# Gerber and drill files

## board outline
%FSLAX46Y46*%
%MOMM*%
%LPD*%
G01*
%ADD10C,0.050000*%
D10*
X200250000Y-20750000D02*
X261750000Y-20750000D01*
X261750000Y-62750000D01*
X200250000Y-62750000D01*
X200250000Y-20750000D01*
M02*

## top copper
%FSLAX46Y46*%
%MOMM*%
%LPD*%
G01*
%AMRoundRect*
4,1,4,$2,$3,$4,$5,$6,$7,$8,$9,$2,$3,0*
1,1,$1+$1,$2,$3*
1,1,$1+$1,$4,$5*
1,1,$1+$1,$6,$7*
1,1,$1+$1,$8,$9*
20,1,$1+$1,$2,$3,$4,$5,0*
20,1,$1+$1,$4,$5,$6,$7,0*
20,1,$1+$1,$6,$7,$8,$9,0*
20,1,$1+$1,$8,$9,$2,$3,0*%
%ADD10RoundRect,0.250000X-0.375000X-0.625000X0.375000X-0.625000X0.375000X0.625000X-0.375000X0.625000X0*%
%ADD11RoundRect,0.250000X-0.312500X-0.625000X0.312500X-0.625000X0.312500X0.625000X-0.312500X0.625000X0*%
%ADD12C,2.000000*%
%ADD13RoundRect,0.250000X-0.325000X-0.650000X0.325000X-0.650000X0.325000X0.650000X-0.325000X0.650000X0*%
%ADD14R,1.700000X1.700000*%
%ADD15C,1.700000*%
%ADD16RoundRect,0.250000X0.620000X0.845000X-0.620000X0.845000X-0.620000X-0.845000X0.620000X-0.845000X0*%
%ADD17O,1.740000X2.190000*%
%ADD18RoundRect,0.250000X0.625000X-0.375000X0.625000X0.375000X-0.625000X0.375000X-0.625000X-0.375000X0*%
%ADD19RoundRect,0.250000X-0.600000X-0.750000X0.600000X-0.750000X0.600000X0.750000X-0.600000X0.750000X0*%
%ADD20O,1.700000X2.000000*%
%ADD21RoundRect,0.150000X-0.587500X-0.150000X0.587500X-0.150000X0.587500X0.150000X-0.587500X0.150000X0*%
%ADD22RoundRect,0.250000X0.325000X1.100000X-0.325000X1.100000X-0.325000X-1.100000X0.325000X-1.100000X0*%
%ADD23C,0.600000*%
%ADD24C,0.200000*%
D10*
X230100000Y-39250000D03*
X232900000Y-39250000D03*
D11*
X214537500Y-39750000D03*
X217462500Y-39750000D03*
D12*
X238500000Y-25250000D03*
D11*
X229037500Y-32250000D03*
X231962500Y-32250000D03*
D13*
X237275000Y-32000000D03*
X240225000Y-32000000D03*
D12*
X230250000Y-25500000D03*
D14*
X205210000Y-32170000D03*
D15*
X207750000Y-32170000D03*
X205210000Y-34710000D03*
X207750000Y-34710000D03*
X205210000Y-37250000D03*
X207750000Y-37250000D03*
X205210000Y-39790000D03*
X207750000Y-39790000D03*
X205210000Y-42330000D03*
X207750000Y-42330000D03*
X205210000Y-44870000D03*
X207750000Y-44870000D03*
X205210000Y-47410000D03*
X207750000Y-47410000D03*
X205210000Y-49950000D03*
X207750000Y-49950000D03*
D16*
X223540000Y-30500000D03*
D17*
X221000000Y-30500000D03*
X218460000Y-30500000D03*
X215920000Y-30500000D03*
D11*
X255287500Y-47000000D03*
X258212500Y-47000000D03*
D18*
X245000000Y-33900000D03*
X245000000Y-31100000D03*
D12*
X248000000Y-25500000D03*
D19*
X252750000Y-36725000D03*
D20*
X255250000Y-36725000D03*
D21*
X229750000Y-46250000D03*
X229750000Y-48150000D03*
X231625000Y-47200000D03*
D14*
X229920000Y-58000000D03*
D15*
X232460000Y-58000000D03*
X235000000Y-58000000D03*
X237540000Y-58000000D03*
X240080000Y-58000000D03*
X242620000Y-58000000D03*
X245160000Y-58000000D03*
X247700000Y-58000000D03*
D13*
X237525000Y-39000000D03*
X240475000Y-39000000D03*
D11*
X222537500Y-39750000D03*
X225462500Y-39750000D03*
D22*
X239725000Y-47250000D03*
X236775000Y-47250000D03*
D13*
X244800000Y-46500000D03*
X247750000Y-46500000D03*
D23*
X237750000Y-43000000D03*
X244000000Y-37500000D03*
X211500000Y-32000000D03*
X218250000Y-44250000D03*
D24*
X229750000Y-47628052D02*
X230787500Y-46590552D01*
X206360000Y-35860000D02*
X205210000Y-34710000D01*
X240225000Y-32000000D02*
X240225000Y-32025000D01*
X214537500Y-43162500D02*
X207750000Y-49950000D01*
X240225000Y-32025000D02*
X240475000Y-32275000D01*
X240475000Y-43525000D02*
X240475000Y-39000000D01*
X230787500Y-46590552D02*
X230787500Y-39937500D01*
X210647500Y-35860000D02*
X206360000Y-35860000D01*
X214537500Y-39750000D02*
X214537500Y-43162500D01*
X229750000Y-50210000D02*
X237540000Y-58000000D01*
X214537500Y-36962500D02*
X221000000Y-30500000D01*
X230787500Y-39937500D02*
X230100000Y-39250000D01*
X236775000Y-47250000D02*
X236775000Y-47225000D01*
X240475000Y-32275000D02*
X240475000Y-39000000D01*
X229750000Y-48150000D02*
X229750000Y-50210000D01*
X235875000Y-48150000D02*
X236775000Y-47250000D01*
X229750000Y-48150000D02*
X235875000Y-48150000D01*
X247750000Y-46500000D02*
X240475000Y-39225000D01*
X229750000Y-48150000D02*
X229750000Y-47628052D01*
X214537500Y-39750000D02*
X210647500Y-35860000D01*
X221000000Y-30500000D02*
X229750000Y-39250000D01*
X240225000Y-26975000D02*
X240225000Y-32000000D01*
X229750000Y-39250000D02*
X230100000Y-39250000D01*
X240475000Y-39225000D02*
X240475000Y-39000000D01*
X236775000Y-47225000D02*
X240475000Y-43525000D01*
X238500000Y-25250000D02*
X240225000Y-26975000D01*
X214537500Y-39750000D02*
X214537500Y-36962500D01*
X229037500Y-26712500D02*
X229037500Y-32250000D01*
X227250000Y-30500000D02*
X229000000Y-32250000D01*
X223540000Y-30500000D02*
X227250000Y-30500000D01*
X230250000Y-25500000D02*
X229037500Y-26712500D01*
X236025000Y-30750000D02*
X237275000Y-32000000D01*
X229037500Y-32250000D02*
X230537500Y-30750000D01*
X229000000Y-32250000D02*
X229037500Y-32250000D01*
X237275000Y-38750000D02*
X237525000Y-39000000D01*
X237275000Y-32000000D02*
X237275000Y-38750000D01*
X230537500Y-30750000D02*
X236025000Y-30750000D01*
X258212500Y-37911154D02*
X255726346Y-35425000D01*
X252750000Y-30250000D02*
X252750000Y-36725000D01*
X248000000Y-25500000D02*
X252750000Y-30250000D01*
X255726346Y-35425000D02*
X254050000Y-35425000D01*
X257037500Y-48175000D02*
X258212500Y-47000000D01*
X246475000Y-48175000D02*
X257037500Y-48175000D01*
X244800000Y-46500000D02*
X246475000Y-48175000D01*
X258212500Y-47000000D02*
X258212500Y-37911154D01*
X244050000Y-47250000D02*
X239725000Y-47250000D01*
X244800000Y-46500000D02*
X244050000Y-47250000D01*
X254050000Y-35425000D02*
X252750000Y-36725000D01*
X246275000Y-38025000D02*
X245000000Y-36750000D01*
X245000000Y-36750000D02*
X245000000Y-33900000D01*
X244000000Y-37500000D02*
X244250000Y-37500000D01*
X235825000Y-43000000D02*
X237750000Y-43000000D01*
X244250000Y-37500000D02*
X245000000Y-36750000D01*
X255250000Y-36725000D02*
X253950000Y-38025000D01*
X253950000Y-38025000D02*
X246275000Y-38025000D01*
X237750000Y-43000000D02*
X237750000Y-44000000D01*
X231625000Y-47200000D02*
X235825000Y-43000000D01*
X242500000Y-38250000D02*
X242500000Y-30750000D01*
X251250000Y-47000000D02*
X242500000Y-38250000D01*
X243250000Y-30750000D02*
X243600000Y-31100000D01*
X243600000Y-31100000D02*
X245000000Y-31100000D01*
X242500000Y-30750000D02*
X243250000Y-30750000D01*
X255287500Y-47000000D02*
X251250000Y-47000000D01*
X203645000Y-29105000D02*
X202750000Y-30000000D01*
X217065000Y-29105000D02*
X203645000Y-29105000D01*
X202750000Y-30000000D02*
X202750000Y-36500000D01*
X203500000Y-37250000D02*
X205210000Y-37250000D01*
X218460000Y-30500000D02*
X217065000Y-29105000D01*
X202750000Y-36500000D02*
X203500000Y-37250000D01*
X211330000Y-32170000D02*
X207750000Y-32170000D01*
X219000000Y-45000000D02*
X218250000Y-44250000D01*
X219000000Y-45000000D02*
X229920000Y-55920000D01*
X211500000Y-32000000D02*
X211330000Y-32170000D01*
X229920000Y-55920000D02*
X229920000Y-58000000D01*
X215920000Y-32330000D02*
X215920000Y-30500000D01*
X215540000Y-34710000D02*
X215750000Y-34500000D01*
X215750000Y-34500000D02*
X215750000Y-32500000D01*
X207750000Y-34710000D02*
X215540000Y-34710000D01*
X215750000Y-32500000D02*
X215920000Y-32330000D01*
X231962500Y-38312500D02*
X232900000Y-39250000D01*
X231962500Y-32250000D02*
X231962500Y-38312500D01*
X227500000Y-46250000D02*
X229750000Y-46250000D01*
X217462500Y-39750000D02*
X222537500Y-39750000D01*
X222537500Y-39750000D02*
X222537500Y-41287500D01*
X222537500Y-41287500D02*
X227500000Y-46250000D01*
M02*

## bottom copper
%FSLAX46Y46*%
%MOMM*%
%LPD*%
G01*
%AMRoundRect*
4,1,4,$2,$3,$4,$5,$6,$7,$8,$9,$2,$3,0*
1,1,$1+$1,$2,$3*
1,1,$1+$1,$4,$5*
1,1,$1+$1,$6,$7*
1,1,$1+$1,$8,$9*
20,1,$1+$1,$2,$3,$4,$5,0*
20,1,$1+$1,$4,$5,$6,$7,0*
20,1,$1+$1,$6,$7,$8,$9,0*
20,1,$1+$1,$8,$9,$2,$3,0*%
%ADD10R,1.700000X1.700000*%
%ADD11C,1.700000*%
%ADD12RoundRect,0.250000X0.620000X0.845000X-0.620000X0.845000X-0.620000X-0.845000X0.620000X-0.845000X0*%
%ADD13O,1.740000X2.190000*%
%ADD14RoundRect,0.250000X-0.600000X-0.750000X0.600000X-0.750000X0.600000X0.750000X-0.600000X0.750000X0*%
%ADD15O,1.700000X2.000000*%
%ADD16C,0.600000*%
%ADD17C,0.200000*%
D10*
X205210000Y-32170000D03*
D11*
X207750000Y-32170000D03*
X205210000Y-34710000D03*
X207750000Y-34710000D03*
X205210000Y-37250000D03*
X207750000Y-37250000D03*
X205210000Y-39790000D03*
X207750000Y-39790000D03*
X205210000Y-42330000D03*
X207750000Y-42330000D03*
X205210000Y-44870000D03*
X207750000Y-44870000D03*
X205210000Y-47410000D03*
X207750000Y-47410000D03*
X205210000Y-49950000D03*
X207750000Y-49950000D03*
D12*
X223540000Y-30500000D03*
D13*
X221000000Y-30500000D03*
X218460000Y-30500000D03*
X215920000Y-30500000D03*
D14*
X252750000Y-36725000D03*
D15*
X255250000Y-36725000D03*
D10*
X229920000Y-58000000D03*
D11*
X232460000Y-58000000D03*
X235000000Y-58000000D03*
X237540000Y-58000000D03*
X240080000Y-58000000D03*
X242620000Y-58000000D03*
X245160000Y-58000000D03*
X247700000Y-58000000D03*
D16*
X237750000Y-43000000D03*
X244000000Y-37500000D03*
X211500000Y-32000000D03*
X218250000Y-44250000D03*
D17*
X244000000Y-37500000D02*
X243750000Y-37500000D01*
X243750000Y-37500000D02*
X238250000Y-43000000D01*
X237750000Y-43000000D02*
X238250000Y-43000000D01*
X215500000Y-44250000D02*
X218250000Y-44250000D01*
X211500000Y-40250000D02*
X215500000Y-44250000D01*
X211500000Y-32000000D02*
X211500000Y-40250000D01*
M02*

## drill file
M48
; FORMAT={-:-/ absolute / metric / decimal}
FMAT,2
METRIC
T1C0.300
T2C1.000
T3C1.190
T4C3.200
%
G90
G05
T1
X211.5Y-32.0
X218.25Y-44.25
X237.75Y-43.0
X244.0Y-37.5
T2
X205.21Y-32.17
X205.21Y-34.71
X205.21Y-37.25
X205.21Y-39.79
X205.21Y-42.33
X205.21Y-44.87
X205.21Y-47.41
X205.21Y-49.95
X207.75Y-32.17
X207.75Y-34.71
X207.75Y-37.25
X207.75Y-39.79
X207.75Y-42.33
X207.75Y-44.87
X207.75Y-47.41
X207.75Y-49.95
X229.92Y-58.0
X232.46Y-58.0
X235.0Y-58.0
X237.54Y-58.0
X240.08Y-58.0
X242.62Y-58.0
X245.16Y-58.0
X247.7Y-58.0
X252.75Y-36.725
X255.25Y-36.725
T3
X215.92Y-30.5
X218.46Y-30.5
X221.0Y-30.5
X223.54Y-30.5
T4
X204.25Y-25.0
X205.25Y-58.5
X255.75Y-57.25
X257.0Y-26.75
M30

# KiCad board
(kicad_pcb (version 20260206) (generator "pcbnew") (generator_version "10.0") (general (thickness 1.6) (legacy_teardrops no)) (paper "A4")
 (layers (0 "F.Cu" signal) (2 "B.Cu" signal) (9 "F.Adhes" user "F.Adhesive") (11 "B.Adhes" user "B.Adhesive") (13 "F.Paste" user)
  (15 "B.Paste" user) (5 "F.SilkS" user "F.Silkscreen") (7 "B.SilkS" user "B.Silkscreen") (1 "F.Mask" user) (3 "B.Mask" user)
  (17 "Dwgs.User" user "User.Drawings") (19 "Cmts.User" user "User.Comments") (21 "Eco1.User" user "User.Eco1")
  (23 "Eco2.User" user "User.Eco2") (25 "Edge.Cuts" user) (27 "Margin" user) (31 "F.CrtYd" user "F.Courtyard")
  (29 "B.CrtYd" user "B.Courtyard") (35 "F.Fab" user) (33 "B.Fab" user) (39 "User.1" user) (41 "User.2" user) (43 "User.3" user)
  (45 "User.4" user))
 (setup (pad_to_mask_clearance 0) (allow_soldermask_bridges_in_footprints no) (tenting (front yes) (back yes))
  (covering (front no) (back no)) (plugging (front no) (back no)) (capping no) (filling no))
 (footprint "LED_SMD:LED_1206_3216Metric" (layer "F.Cu") (at 231.5 39.25)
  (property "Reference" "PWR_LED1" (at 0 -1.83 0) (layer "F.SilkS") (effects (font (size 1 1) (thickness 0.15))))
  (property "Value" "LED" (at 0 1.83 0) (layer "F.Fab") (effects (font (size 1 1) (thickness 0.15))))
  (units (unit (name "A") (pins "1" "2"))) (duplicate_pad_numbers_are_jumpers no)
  (pad "1" smd roundrect (at -1.4 0) (size 1.25 1.75) (layers "F.Cu" "F.Mask" "F.Paste") (roundrect_rratio 0.2) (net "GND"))
  (pad "2" smd roundrect (at 1.4 0) (size 1.25 1.75) (layers "F.Cu" "F.Mask" "F.Paste") (roundrect_rratio 0.2) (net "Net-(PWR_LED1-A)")))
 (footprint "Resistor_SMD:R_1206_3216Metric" (layer "F.Cu") (at 216 39.75)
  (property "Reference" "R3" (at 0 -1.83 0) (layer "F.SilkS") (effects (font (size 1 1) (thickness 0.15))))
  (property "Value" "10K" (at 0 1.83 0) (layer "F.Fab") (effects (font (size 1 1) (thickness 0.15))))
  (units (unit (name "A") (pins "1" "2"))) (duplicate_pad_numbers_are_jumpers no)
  (pad "1" smd roundrect (at -1.4625 0) (size 1.125 1.75) (layers "F.Cu" "F.Mask" "F.Paste") (roundrect_rratio 0.222222) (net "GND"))
  (pad "2" smd roundrect (at 1.4625 0) (size 1.125 1.75) (layers "F.Cu" "F.Mask" "F.Paste") (roundrect_rratio 0.222222) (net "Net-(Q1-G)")))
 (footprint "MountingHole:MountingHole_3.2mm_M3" (layer "F.Cu") (at 255.75 57.25)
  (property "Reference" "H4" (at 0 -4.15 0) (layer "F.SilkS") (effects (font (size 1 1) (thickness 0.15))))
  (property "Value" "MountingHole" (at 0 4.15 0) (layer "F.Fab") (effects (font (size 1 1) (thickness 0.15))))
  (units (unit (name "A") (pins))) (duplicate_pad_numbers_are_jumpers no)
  (pad "" np_thru_hole circle (at 0 0) (size 3.2 3.2) (drill 3.2) (layers "*.Cu" "*.Mask")))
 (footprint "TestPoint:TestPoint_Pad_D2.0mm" (layer "F.Cu") (at 238.5 25.25 180)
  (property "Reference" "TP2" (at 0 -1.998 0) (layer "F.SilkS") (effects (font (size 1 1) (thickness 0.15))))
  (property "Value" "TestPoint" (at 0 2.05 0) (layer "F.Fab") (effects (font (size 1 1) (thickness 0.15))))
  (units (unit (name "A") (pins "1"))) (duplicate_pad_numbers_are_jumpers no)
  (pad "1" smd circle (at 0 0 180) (size 2 2) (layers "F.Cu" "F.Mask") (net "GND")))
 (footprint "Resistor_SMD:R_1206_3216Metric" (layer "F.Cu") (at 230.5 32.25)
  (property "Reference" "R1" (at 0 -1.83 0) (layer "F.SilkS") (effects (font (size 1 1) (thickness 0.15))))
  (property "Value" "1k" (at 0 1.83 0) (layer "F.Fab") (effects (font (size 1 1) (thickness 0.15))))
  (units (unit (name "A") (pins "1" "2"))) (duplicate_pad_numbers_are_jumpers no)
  (pad "1" smd roundrect (at -1.4625 0) (size 1.125 1.75) (layers "F.Cu" "F.Mask" "F.Paste") (roundrect_rratio 0.222222) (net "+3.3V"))
  (pad "2" smd roundrect (at 1.4625 0) (size 1.125 1.75) (layers "F.Cu" "F.Mask" "F.Paste") (roundrect_rratio 0.222222)
   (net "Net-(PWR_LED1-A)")))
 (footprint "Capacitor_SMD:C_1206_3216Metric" (layer "F.Cu") (at 238.75 32)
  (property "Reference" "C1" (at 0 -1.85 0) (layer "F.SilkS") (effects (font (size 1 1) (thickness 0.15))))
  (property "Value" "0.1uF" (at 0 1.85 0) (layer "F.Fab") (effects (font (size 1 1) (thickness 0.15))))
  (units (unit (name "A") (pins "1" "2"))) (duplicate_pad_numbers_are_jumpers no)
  (pad "1" smd roundrect (at -1.475 0) (size 1.15 1.8) (layers "F.Cu" "F.Mask" "F.Paste") (roundrect_rratio 0.217391) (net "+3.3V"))
  (pad "2" smd roundrect (at 1.475 0) (size 1.15 1.8) (layers "F.Cu" "F.Mask" "F.Paste") (roundrect_rratio 0.217391) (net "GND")))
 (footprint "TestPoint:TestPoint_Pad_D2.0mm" (layer "F.Cu") (at 230.25 25.5 180)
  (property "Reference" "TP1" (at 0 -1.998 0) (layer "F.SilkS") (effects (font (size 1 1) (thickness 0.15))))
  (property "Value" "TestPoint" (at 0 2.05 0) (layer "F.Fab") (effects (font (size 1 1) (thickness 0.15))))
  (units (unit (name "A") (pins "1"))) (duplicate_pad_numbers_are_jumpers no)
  (pad "1" smd circle (at 0 0 180) (size 2 2) (layers "F.Cu" "F.Mask") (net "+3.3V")))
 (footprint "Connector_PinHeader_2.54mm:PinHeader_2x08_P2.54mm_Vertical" (layer "F.Cu") (at 205.21 32.17)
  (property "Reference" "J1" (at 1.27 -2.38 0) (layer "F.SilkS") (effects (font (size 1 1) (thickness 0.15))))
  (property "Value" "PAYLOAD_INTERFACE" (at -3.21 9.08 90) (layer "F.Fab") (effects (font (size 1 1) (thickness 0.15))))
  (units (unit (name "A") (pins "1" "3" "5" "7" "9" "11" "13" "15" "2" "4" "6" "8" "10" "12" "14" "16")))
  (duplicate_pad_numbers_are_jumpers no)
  (pad "1" thru_hole rect (at 0 0) (size 1.7 1.7) (drill 1) (layers "*.Cu" "*.Mask") (remove_unused_layers no) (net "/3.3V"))
  (pad "2" thru_hole circle (at 2.54 0) (size 1.7 1.7) (drill 1) (layers "*.Cu" "*.Mask") (remove_unused_layers no) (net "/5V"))
  (pad "3" thru_hole circle (at 0 2.54) (size 1.7 1.7) (drill 1) (layers "*.Cu" "*.Mask") (remove_unused_layers no) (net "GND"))
  (pad "4" thru_hole circle (at 2.54 2.54) (size 1.7 1.7) (drill 1) (layers "*.Cu" "*.Mask") (remove_unused_layers no) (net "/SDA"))
  (pad "5" thru_hole circle (at 0 5.08) (size 1.7 1.7) (drill 1) (layers "*.Cu" "*.Mask") (remove_unused_layers no) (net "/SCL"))
  (pad "6" thru_hole circle (at 2.54 5.08) (size 1.7 1.7) (drill 1) (layers "*.Cu" "*.Mask") (remove_unused_layers no) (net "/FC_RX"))
  (pad "7" thru_hole circle (at 0 7.62) (size 1.7 1.7) (drill 1) (layers "*.Cu" "*.Mask") (remove_unused_layers no) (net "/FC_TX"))
  (pad "8" thru_hole circle (at 2.54 7.62) (size 1.7 1.7) (drill 1) (layers "*.Cu" "*.Mask") (remove_unused_layers no) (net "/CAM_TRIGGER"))
  (pad "9" thru_hole circle (at 0 10.16) (size 1.7 1.7) (drill 1) (layers "*.Cu" "*.Mask") (remove_unused_layers no) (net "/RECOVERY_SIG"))
  (pad "10" thru_hole circle (at 2.54 10.16) (size 1.7 1.7) (drill 1) (layers "*.Cu" "*.Mask") (remove_unused_layers no)
   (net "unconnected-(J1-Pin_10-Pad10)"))
  (pad "11" thru_hole circle (at 0 12.7) (size 1.7 1.7) (drill 1) (layers "*.Cu" "*.Mask") (remove_unused_layers no)
   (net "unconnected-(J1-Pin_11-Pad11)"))
  (pad "12" thru_hole circle (at 2.54 12.7) (size 1.7 1.7) (drill 1) (layers "*.Cu" "*.Mask") (remove_unused_layers no)
   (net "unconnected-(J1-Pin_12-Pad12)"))
  (pad "13" thru_hole circle (at 0 15.24) (size 1.7 1.7) (drill 1) (layers "*.Cu" "*.Mask") (remove_unused_layers no)
   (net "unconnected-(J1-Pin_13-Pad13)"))
  (pad "14" thru_hole circle (at 2.54 15.24) (size 1.7 1.7) (drill 1) (layers "*.Cu" "*.Mask") (remove_unused_layers no)
   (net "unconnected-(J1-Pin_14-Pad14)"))
  (pad "15" thru_hole circle (at 0 17.78) (size 1.7 1.7) (drill 1) (layers "*.Cu" "*.Mask") (remove_unused_layers no)
   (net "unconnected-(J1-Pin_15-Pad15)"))
  (pad "16" thru_hole circle (at 2.54 17.78) (size 1.7 1.7) (drill 1) (layers "*.Cu" "*.Mask") (remove_unused_layers no) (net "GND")))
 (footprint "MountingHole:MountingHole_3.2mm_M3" (layer "F.Cu") (at 205.25 58.5)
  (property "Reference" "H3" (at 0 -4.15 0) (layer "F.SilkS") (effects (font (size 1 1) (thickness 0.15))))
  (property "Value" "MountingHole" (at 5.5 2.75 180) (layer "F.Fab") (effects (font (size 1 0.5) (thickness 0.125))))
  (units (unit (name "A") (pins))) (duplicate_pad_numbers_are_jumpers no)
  (pad "" np_thru_hole circle (at 0 0) (size 3.2 3.2) (drill 3.2) (layers "*.Cu" "*.Mask")))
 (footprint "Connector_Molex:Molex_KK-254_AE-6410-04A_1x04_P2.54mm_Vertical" (layer "F.Cu") (at 223.54 30.5 180)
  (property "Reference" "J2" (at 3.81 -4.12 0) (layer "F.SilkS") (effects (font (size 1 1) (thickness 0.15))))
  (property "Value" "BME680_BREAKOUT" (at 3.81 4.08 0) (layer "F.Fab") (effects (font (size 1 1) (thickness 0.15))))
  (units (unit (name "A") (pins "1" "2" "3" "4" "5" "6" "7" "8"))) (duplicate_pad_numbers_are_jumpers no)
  (pad "1" thru_hole roundrect (at 0 0 180) (size 1.74 2.19) (drill 1.19) (layers "*.Cu" "*.Mask") (remove_unused_layers no)
   (roundrect_rratio 0.143678) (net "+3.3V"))
  (pad "2" thru_hole oval (at 2.54 0 180) (size 1.74 2.19) (drill 1.19) (layers "*.Cu" "*.Mask") (remove_unused_layers no) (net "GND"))
  (pad "3" thru_hole oval (at 5.08 0 180) (size 1.74 2.19) (drill 1.19) (layers "*.Cu" "*.Mask") (remove_unused_layers no) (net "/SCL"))
  (pad "4" thru_hole oval (at 7.62 0 180) (size 1.74 2.19) (drill 1.19) (layers "*.Cu" "*.Mask") (remove_unused_layers no) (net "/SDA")))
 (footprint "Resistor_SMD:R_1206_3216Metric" (layer "F.Cu") (at 256.75 47)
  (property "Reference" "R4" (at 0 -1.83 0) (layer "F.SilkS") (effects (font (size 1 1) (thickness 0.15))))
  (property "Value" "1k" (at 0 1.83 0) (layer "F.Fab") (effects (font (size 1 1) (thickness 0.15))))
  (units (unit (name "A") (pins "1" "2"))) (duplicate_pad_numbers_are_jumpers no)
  (pad "1" smd roundrect (at -1.4625 0) (size 1.125 1.75) (layers "F.Cu" "F.Mask" "F.Paste") (roundrect_rratio 0.222222) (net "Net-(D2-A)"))
  (pad "2" smd roundrect (at 1.4625 0) (size 1.125 1.75) (layers "F.Cu" "F.Mask" "F.Paste") (roundrect_rratio 0.222222) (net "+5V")))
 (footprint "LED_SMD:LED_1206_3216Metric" (layer "F.Cu") (at 245 32.5 90)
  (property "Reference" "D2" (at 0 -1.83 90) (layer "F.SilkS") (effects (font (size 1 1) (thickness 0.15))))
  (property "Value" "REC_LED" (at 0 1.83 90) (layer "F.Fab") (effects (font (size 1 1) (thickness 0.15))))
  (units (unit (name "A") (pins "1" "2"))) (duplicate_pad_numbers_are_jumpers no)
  (pad "1" smd roundrect (at -1.4 0 90) (size 1.25 1.75) (layers "F.Cu" "F.Mask" "F.Paste") (roundrect_rratio 0.2) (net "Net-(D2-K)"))
  (pad "2" smd roundrect (at 1.4 0 90) (size 1.25 1.75) (layers "F.Cu" "F.Mask" "F.Paste") (roundrect_rratio 0.2) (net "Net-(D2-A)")))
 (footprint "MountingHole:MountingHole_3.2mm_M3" (layer "F.Cu") (at 204.25 25)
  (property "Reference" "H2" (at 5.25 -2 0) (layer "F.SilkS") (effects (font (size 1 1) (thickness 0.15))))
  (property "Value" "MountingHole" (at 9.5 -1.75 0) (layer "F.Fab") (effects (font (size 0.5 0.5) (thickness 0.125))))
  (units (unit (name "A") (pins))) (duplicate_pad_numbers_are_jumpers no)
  (pad "" np_thru_hole circle (at 0 0) (size 3.2 3.2) (drill 3.2) (layers "*.Cu" "*.Mask")))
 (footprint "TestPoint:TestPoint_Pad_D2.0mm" (layer "F.Cu") (at 248 25.5 180)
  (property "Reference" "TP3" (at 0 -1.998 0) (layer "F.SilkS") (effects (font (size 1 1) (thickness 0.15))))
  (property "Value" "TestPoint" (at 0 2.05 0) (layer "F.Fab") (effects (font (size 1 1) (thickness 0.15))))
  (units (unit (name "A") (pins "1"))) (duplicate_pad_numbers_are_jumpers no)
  (pad "1" smd circle (at 0 0 180) (size 2 2) (layers "F.Cu" "F.Mask") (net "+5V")))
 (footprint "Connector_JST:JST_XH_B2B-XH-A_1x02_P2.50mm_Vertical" (layer "F.Cu") (at 252.75 36.725)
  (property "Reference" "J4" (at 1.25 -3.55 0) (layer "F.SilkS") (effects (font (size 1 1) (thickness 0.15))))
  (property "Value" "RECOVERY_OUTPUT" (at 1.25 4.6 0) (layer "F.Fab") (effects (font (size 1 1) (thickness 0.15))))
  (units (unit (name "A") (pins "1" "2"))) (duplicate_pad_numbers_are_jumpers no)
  (pad "1" thru_hole roundrect (at 0 0) (size 1.7 2) (drill 1) (layers "*.Cu" "*.Mask") (remove_unused_layers no)
   (roundrect_rratio 0.147059) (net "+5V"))
  (pad "2" thru_hole oval (at 2.5 0) (size 1.7 2) (drill 1) (layers "*.Cu" "*.Mask") (remove_unused_layers no) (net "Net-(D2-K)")))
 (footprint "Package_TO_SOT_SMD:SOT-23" (layer "F.Cu") (at 230.6875 47.2)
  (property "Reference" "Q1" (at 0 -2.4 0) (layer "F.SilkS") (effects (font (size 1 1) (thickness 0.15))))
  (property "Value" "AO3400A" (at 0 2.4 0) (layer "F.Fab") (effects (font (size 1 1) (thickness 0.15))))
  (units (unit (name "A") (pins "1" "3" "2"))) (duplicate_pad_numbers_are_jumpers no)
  (pad "1" smd roundrect (at -0.9375 -0.95) (size 1.475 0.6) (layers "F.Cu" "F.Mask" "F.Paste") (roundrect_rratio 0.25) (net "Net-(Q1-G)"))
  (pad "2" smd roundrect (at -0.9375 0.95) (size 1.475 0.6) (layers "F.Cu" "F.Mask" "F.Paste") (roundrect_rratio 0.25) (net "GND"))
  (pad "3" smd roundrect (at 0.9375 0) (size 1.475 0.6) (layers "F.Cu" "F.Mask" "F.Paste") (roundrect_rratio 0.25) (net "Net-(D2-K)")))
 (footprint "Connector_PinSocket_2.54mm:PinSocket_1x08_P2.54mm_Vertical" (layer "F.Cu") (at 229.92 58 90)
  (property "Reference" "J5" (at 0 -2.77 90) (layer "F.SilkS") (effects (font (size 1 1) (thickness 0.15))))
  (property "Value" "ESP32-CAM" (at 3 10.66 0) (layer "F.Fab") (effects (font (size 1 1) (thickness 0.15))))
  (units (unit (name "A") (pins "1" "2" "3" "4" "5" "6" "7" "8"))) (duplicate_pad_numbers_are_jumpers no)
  (pad "1" thru_hole rect (at 0 0 90) (size 1.7 1.7) (drill 1) (layers "*.Cu" "*.Mask") (remove_unused_layers no) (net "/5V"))
  (pad "2" thru_hole circle (at 0 2.54 90) (size 1.7 1.7) (drill 1) (layers "*.Cu" "*.Mask") (remove_unused_layers no)
   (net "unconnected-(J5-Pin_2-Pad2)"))
  (pad "3" thru_hole circle (at 0 5.08 90) (size 1.7 1.7) (drill 1) (layers "*.Cu" "*.Mask") (remove_unused_layers no)
   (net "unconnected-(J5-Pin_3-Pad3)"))
  (pad "4" thru_hole circle (at 0 7.62 90) (size 1.7 1.7) (drill 1) (layers "*.Cu" "*.Mask") (remove_unused_layers no) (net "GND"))
  (pad "5" thru_hole circle (at 0 10.16 90) (size 1.7 1.7) (drill 1) (layers "*.Cu" "*.Mask") (remove_unused_layers no) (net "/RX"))
  (pad "6" thru_hole circle (at 0 12.7 90) (size 1.7 1.7) (drill 1) (layers "*.Cu" "*.Mask") (remove_unused_layers no) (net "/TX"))
  (pad "7" thru_hole circle (at 0 15.24 90) (size 1.7 1.7) (drill 1) (layers "*.Cu" "*.Mask") (remove_unused_layers no)
   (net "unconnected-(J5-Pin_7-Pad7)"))
  (pad "8" thru_hole circle (at 0 17.78 90) (size 1.7 1.7) (drill 1) (layers "*.Cu" "*.Mask") (remove_unused_layers no)
   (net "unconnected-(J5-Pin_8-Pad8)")))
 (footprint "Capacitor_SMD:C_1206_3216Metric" (layer "F.Cu") (at 239 39)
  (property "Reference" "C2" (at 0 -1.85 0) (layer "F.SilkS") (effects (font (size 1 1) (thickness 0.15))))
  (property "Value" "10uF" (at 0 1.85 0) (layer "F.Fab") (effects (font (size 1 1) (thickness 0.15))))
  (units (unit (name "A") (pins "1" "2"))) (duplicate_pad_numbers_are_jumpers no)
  (pad "1" smd roundrect (at -1.475 0) (size 1.15 1.8) (layers "F.Cu" "F.Mask" "F.Paste") (roundrect_rratio 0.217391) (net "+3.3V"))
  (pad "2" smd roundrect (at 1.475 0) (size 1.15 1.8) (layers "F.Cu" "F.Mask" "F.Paste") (roundrect_rratio 0.217391) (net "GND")))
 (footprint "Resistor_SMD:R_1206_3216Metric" (layer "F.Cu") (at 224 39.75)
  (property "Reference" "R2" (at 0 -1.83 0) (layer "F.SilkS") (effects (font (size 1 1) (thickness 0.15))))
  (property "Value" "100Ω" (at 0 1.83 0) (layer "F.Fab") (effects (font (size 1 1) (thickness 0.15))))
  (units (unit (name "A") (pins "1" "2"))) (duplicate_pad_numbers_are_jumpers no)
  (pad "1" smd roundrect (at -1.4625 0) (size 1.125 1.75) (layers "F.Cu" "F.Mask" "F.Paste") (roundrect_rratio 0.222222) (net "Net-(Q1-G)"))
  (pad "2" smd roundrect (at 1.4625 0) (size 1.125 1.75) (layers "F.Cu" "F.Mask" "F.Paste") (roundrect_rratio 0.222222)
   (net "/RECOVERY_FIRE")))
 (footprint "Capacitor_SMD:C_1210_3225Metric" (layer "F.Cu") (at 238.25 47.25 180)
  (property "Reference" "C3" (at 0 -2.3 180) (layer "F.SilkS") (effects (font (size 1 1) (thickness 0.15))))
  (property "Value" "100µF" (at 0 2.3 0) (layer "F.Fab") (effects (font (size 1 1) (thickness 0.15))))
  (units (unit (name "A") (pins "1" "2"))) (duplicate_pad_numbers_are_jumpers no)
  (pad "1" smd roundrect (at -1.475 0 180) (size 1.15 2.7) (layers "F.Cu" "F.Mask" "F.Paste") (roundrect_rratio 0.217391) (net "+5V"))
  (pad "2" smd roundrect (at 1.475 0 180) (size 1.15 2.7) (layers "F.Cu" "F.Mask" "F.Paste") (roundrect_rratio 0.217391) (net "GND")))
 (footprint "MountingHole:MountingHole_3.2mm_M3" (layer "F.Cu") (at 257 26.75)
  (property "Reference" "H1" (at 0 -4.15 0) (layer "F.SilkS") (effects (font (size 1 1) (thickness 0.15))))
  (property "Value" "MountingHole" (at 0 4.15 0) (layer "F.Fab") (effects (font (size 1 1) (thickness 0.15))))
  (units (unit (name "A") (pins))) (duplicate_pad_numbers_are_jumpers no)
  (pad "" np_thru_hole circle (at 0 0) (size 3.2 3.2) (drill 3.2) (layers "*.Cu" "*.Mask")))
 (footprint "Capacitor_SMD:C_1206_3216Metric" (layer "F.Cu") (at 246.275 46.5)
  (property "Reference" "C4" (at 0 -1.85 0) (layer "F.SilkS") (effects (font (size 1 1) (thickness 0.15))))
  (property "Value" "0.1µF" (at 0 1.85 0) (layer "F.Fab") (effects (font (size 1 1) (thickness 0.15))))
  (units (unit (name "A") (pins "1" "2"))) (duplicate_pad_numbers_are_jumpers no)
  (pad "1" smd roundrect (at -1.475 0) (size 1.15 1.8) (layers "F.Cu" "F.Mask" "F.Paste") (roundrect_rratio 0.217391) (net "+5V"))
  (pad "2" smd roundrect (at 1.475 0) (size 1.15 1.8) (layers "F.Cu" "F.Mask" "F.Paste") (roundrect_rratio 0.217391) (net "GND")))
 (gr_rect (start 200.25 20.75) (end 261.75 62.75) (stroke (width 0.05) (type default)) (fill no) (layer "Edge.Cuts"))
 (segment (start 229.75 47.628052) (end 230.7875 46.590552) (width 0.2) (layer "F.Cu") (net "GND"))
 (segment (start 206.36 35.86) (end 205.21 34.71) (width 0.2) (layer "F.Cu") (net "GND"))
 (segment (start 240.225 32) (end 240.225 32.025) (width 0.2) (layer "F.Cu") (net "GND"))
 (segment (start 214.5375 43.1625) (end 207.75 49.95) (width 0.2) (layer "F.Cu") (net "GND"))
 (segment (start 240.225 32.025) (end 240.475 32.275) (width 0.2) (layer "F.Cu") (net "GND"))
 (segment (start 240.475 43.525) (end 240.475 39) (width 0.2) (layer "F.Cu") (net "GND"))
 (segment (start 230.7875 46.590552) (end 230.7875 39.9375) (width 0.2) (layer "F.Cu") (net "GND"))
 (segment (start 210.6475 35.86) (end 206.36 35.86) (width 0.2) (layer "F.Cu") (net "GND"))
 (segment (start 214.5375 39.75) (end 214.5375 43.1625) (width 0.2) (layer "F.Cu") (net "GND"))
 (segment (start 229.75 50.21) (end 237.54 58) (width 0.2) (layer "F.Cu") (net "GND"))
 (segment (start 214.5375 36.9625) (end 221 30.5) (width 0.2) (layer "F.Cu") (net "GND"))
 (segment (start 230.7875 39.9375) (end 230.1 39.25) (width 0.2) (layer "F.Cu") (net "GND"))
 (segment (start 236.775 47.25) (end 236.775 47.225) (width 0.2) (layer "F.Cu") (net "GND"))
 (segment (start 240.475 32.275) (end 240.475 39) (width 0.2) (layer "F.Cu") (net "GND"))
 (segment (start 229.75 48.15) (end 229.75 50.21) (width 0.2) (layer "F.Cu") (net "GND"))
 (segment (start 235.875 48.15) (end 236.775 47.25) (width 0.2) (layer "F.Cu") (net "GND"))
 (segment (start 229.75 48.15) (end 235.875 48.15) (width 0.2) (layer "F.Cu") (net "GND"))
 (segment (start 247.75 46.5) (end 240.475 39.225) (width 0.2) (layer "F.Cu") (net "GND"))
 (segment (start 229.75 48.15) (end 229.75 47.628052) (width 0.2) (layer "F.Cu") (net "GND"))
 (segment (start 214.5375 39.75) (end 210.6475 35.86) (width 0.2) (layer "F.Cu") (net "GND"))
 (segment (start 221 30.5) (end 229.75 39.25) (width 0.2) (layer "F.Cu") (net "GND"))
 (segment (start 240.225 26.975) (end 240.225 32) (width 0.2) (layer "F.Cu") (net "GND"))
 (segment (start 229.75 39.25) (end 230.1 39.25) (width 0.2) (layer "F.Cu") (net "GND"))
 (segment (start 240.475 39.225) (end 240.475 39) (width 0.2) (layer "F.Cu") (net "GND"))
 (segment (start 236.775 47.225) (end 240.475 43.525) (width 0.2) (layer "F.Cu") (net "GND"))
 (segment (start 238.5 25.25) (end 240.225 26.975) (width 0.2) (layer "F.Cu") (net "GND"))
 (segment (start 214.5375 39.75) (end 214.5375 36.9625) (width 0.2) (layer "F.Cu") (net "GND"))
 (segment (start 229.0375 26.7125) (end 229.0375 32.25) (width 0.2) (layer "F.Cu") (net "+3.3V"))
 (segment (start 227.25 30.5) (end 229 32.25) (width 0.2) (layer "F.Cu") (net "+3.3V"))
 (segment (start 223.54 30.5) (end 227.25 30.5) (width 0.2) (layer "F.Cu") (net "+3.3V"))
 (segment (start 230.25 25.5) (end 229.0375 26.7125) (width 0.2) (layer "F.Cu") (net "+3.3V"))
 (segment (start 236.025 30.75) (end 237.275 32) (width 0.2) (layer "F.Cu") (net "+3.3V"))
 (segment (start 229.0375 32.25) (end 230.5375 30.75) (width 0.2) (layer "F.Cu") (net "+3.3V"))
 (segment (start 229 32.25) (end 229.0375 32.25) (width 0.2) (layer "F.Cu") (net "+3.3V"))
 (segment (start 237.275 38.75) (end 237.525 39) (width 0.2) (layer "F.Cu") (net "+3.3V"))
 (segment (start 237.275 32) (end 237.275 38.75) (width 0.2) (layer "F.Cu") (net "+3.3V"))
 (segment (start 230.5375 30.75) (end 236.025 30.75) (width 0.2) (layer "F.Cu") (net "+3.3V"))
 (segment (start 258.2125 37.911154) (end 255.726346 35.425) (width 0.2) (layer "F.Cu") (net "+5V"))
 (segment (start 252.75 30.25) (end 252.75 36.725) (width 0.2) (layer "F.Cu") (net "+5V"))
 (segment (start 248 25.5) (end 252.75 30.25) (width 0.2) (layer "F.Cu") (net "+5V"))
 (segment (start 255.726346 35.425) (end 254.05 35.425) (width 0.2) (layer "F.Cu") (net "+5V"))
 (segment (start 257.0375 48.175) (end 258.2125 47) (width 0.2) (layer "F.Cu") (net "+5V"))
 (segment (start 246.475 48.175) (end 257.0375 48.175) (width 0.2) (layer "F.Cu") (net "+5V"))
 (segment (start 244.8 46.5) (end 246.475 48.175) (width 0.2) (layer "F.Cu") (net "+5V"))
 (segment (start 258.2125 47) (end 258.2125 37.911154) (width 0.2) (layer "F.Cu") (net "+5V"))
 (segment (start 244.05 47.25) (end 239.725 47.25) (width 0.2) (layer "F.Cu") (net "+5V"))
 (segment (start 244.8 46.5) (end 244.05 47.25) (width 0.2) (layer "F.Cu") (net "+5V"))
 (segment (start 254.05 35.425) (end 252.75 36.725) (width 0.2) (layer "F.Cu") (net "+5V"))
 (segment (start 246.275 38.025) (end 245 36.75) (width 0.2) (layer "F.Cu") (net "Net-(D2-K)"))
 (segment (start 245 36.75) (end 245 33.9) (width 0.2) (layer "F.Cu") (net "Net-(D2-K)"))
 (segment (start 244 37.5) (end 244.25 37.5) (width 0.2) (layer "F.Cu") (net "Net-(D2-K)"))
 (segment (start 235.825 43) (end 237.75 43) (width 0.2) (layer "F.Cu") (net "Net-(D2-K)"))
 (segment (start 244.25 37.5) (end 245 36.75) (width 0.2) (layer "F.Cu") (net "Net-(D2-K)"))
 (segment (start 255.25 36.725) (end 253.95 38.025) (width 0.2) (layer "F.Cu") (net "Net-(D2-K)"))
 (segment (start 253.95 38.025) (end 246.275 38.025) (width 0.2) (layer "F.Cu") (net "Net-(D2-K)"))
 (segment (start 237.75 43) (end 237.75 44) (width 0.2) (layer "F.Cu") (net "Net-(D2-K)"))
 (segment (start 231.625 47.2) (end 235.825 43) (width 0.2) (layer "F.Cu") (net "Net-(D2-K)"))
 (via (at 237.75 43) (size 0.6) (drill 0.3) (layers "F.Cu" "B.Cu") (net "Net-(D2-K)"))
 (via (at 244 37.5) (size 0.6) (drill 0.3) (layers "F.Cu" "B.Cu") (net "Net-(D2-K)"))
 (segment (start 244 37.5) (end 243.75 37.5) (width 0.2) (layer "B.Cu") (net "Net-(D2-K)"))
 (segment (start 243.75 37.5) (end 238.25 43) (width 0.2) (layer "B.Cu") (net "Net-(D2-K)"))
 (segment (start 237.75 43) (end 238.25 43) (width 0.2) (layer "B.Cu") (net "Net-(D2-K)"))
 (segment (start 242.5 38.25) (end 242.5 30.75) (width 0.2) (layer "F.Cu") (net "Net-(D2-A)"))
 (segment (start 251.25 47) (end 242.5 38.25) (width 0.2) (layer "F.Cu") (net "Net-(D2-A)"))
 (segment (start 243.25 30.75) (end 243.6 31.1) (width 0.2) (layer "F.Cu") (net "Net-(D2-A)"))
 (segment (start 243.6 31.1) (end 245 31.1) (width 0.2) (layer "F.Cu") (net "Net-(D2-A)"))
 (segment (start 242.5 30.75) (end 243.25 30.75) (width 0.2) (layer "F.Cu") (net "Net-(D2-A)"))
 (segment (start 255.2875 47) (end 251.25 47) (width 0.2) (layer "F.Cu") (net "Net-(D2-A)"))
 (segment (start 203.645 29.105) (end 202.75 30) (width 0.2) (layer "F.Cu") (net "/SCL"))
 (segment (start 217.065 29.105) (end 203.645 29.105) (width 0.2) (layer "F.Cu") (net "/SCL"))
 (segment (start 202.75 30) (end 202.75 36.5) (width 0.2) (layer "F.Cu") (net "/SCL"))
 (segment (start 203.5 37.25) (end 205.21 37.25) (width 0.2) (layer "F.Cu") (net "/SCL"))
 (segment (start 218.46 30.5) (end 217.065 29.105) (width 0.2) (layer "F.Cu") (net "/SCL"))
 (segment (start 202.75 36.5) (end 203.5 37.25) (width 0.2) (layer "F.Cu") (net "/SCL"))
 (segment (start 211.33 32.17) (end 207.75 32.17) (width 0.2) (layer "F.Cu") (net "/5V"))
 (segment (start 219 45) (end 218.25 44.25) (width 0.2) (layer "F.Cu") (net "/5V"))
 (segment (start 219 45) (end 229.92 55.92) (width 0.2) (layer "F.Cu") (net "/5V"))
 (segment (start 211.5 32) (end 211.33 32.17) (width 0.2) (layer "F.Cu") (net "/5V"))
 (segment (start 229.92 55.92) (end 229.92 58) (width 0.2) (layer "F.Cu") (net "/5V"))
 (via (at 211.5 32) (size 0.6) (drill 0.3) (layers "F.Cu" "B.Cu") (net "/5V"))
 (via (at 218.25 44.25) (size 0.6) (drill 0.3) (layers "F.Cu" "B.Cu") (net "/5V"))
 (segment (start 215.5 44.25) (end 218.25 44.25) (width 0.2) (layer "B.Cu") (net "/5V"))
 (segment (start 211.5 40.25) (end 215.5 44.25) (width 0.2) (layer "B.Cu") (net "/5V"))
 (segment (start 211.5 32) (end 211.5 40.25) (width 0.2) (layer "B.Cu") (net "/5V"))
 (segment (start 215.92 32.33) (end 215.92 30.5) (width 0.2) (layer "F.Cu") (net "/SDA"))
 (segment (start 215.54 34.71) (end 215.75 34.5) (width 0.2) (layer "F.Cu") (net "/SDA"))
 (segment (start 215.75 34.5) (end 215.75 32.5) (width 0.2) (layer "F.Cu") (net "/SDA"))
 (segment (start 207.75 34.71) (end 215.54 34.71) (width 0.2) (layer "F.Cu") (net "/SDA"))
 (segment (start 215.75 32.5) (end 215.92 32.33) (width 0.2) (layer "F.Cu") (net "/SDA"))
 (segment (start 231.9625 38.3125) (end 232.9 39.25) (width 0.2) (layer "F.Cu") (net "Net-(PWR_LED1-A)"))
 (segment (start 231.9625 32.25) (end 231.9625 38.3125) (width 0.2) (layer "F.Cu") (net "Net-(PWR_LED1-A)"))
 (segment (start 227.5 46.25) (end 229.75 46.25) (width 0.2) (layer "F.Cu") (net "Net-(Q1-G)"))
 (segment (start 217.4625 39.75) (end 222.5375 39.75) (width 0.2) (layer "F.Cu") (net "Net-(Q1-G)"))
 (segment (start 222.5375 39.75) (end 222.5375 41.2875) (width 0.2) (layer "F.Cu") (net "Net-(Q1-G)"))
 (segment (start 222.5375 41.2875) (end 227.5 46.25) (width 0.2) (layer "F.Cu") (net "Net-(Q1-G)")))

